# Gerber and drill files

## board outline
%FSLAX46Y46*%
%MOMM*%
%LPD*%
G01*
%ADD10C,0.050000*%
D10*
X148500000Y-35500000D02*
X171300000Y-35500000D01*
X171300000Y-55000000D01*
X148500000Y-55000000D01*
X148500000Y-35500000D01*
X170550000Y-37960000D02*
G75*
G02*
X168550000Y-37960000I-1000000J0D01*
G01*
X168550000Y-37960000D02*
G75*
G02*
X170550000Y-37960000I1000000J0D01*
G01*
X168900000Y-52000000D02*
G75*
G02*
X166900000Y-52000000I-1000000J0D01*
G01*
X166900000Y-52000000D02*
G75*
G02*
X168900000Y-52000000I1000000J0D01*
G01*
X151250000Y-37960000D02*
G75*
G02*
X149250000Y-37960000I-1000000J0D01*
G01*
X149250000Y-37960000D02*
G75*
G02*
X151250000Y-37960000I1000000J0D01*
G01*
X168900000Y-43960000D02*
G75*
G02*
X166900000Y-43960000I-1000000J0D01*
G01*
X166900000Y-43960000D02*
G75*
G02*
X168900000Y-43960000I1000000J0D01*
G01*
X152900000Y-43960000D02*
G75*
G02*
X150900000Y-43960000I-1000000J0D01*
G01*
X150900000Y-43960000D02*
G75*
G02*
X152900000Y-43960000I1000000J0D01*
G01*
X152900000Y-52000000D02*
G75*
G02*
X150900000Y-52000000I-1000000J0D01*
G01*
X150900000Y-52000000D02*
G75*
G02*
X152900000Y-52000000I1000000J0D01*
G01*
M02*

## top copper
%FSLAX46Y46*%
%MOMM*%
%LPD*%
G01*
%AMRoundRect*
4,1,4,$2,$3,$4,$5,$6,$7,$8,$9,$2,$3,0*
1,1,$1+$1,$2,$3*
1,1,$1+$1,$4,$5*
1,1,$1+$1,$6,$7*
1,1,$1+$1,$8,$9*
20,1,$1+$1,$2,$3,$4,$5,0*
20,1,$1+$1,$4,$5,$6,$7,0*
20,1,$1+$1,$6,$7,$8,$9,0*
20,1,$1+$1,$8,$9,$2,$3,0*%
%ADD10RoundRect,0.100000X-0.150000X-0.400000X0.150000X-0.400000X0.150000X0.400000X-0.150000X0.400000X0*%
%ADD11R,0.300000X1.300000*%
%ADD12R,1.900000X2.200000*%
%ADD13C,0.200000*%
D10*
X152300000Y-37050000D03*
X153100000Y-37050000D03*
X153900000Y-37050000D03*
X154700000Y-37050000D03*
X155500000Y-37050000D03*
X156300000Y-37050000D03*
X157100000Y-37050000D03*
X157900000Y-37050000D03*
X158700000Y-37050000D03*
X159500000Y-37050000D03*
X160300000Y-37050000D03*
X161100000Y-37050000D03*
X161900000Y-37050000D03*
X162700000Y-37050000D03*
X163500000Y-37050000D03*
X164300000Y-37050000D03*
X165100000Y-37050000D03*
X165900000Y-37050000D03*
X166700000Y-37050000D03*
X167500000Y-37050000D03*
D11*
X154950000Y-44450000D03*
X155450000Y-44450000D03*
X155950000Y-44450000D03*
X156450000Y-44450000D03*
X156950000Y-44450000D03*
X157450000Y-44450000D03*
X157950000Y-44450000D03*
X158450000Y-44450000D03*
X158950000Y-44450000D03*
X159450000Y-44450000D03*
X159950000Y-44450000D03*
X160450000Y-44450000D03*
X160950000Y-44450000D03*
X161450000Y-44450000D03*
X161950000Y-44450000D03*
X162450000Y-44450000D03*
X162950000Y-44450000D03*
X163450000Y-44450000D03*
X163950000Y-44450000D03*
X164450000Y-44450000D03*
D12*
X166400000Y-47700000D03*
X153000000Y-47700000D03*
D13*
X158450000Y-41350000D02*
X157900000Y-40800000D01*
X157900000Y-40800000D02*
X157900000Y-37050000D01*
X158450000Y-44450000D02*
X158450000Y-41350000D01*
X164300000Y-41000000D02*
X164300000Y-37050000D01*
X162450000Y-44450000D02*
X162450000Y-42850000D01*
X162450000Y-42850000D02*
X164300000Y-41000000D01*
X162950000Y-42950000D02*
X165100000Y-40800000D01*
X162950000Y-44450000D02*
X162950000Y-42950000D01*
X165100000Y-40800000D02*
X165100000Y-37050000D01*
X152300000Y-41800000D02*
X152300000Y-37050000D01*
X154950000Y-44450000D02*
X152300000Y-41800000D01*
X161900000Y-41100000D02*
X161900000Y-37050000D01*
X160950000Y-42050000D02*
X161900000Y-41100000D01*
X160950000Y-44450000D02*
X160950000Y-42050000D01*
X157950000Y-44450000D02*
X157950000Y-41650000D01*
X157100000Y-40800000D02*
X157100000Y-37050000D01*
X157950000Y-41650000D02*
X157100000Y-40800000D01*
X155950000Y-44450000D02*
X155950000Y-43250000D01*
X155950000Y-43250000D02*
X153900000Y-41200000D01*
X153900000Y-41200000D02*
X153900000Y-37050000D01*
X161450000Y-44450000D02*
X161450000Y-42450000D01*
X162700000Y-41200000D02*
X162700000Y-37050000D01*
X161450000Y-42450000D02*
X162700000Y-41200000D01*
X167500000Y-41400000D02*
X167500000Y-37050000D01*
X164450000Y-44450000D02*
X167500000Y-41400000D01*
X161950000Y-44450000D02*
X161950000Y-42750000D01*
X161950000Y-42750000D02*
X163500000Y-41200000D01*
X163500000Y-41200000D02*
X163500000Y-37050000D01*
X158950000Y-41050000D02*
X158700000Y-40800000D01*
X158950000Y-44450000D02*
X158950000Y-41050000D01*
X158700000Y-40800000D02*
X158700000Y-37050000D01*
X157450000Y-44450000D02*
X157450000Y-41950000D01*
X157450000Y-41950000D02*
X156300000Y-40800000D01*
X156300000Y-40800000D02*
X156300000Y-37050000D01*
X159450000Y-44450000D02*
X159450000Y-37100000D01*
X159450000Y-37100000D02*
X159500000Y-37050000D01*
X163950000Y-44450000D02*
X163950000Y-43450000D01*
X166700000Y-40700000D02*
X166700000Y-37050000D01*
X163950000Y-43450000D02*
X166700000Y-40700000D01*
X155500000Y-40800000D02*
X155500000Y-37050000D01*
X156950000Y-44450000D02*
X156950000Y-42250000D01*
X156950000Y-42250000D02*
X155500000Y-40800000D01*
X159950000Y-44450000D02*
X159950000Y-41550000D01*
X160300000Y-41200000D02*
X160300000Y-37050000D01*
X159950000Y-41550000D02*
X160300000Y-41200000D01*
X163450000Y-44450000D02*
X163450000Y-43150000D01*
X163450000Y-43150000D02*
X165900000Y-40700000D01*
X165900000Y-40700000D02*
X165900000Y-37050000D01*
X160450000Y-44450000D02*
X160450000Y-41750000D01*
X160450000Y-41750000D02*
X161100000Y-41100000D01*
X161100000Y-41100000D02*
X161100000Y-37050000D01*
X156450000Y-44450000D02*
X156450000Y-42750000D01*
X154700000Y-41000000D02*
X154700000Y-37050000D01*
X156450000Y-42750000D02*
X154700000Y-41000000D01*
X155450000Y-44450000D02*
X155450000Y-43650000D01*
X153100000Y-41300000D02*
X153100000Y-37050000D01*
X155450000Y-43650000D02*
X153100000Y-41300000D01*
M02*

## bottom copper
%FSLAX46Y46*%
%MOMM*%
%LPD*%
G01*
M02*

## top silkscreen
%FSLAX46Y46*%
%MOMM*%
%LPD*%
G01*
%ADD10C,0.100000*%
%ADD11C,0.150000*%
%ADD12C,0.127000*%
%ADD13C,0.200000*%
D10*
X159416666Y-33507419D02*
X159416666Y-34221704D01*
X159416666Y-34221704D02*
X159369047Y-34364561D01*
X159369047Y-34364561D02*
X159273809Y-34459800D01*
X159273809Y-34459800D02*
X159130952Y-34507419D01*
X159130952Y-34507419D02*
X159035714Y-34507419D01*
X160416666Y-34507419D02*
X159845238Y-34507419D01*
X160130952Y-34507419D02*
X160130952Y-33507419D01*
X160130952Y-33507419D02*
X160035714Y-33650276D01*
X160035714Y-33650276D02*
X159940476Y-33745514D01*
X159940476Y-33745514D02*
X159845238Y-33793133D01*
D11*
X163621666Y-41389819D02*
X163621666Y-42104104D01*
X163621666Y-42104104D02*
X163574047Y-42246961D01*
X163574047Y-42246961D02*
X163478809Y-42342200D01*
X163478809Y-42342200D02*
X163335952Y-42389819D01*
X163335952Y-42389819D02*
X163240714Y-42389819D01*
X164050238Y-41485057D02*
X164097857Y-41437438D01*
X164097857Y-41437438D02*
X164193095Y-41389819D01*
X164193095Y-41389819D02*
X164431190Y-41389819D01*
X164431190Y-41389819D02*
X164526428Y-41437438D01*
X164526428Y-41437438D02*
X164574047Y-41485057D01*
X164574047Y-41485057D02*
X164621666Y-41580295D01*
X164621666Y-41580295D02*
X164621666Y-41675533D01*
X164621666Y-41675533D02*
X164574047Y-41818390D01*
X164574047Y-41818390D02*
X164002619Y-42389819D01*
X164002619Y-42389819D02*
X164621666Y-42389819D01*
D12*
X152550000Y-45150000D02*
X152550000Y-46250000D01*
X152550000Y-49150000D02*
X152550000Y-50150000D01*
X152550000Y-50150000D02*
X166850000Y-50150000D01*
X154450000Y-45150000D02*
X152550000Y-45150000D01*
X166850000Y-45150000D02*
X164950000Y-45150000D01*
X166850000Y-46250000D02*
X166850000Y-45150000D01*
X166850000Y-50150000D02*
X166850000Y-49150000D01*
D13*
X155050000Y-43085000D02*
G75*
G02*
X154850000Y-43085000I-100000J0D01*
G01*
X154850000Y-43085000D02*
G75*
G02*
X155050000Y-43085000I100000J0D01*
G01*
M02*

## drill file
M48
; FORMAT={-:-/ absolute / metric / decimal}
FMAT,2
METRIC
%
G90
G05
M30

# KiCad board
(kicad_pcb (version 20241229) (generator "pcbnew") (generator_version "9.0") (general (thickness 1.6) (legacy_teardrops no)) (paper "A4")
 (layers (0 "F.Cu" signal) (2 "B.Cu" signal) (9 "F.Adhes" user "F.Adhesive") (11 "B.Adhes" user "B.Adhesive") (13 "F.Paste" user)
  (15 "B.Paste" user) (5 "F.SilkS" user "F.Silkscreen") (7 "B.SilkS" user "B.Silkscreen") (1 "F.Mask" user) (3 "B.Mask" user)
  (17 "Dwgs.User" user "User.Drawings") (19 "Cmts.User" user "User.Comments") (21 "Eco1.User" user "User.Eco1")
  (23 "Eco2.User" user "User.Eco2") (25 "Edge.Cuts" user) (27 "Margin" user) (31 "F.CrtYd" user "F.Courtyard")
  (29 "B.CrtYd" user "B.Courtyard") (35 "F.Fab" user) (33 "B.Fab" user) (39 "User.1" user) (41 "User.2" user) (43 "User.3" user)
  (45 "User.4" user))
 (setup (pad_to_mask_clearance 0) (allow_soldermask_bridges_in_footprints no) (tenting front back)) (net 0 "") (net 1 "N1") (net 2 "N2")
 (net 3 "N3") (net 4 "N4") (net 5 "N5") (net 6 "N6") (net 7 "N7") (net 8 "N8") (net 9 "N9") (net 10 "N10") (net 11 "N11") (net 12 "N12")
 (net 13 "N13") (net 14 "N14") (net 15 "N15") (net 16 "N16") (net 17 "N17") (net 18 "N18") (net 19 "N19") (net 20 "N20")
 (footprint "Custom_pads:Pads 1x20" (layer "F.Cu") (at 159.75 37.05)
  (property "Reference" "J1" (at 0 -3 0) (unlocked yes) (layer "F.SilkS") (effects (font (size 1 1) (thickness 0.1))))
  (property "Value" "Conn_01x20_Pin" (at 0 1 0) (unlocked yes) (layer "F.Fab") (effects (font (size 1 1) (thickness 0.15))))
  (pad "1" smd roundrect (at -7.45 0) (size 0.5 1) (layers "F.Cu" "F.Mask" "F.Paste") (roundrect_rratio 0.2) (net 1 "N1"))
  (pad "2" smd roundrect (at -6.65 0) (size 0.5 1) (layers "F.Cu" "F.Mask" "F.Paste") (roundrect_rratio 0.2) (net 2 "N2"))
  (pad "3" smd roundrect (at -5.85 0) (size 0.5 1) (layers "F.Cu" "F.Mask" "F.Paste") (roundrect_rratio 0.2) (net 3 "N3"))
  (pad "4" smd roundrect (at -5.05 0) (size 0.5 1) (layers "F.Cu" "F.Mask" "F.Paste") (roundrect_rratio 0.2) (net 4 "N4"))
  (pad "5" smd roundrect (at -4.25 0) (size 0.5 1) (layers "F.Cu" "F.Mask" "F.Paste") (roundrect_rratio 0.2) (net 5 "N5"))
  (pad "6" smd roundrect (at -3.45 0) (size 0.5 1) (layers "F.Cu" "F.Mask" "F.Paste") (roundrect_rratio 0.2) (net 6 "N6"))
  (pad "7" smd roundrect (at -2.65 0) (size 0.5 1) (layers "F.Cu" "F.Mask" "F.Paste") (roundrect_rratio 0.2) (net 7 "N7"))
  (pad "8" smd roundrect (at -1.85 0) (size 0.5 1) (layers "F.Cu" "F.Mask" "F.Paste") (roundrect_rratio 0.2) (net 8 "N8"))
  (pad "9" smd roundrect (at -1.05 0) (size 0.5 1) (layers "F.Cu" "F.Mask" "F.Paste") (roundrect_rratio 0.2) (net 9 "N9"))
  (pad "10" smd roundrect (at -0.25 0) (size 0.5 1) (layers "F.Cu" "F.Mask" "F.Paste") (roundrect_rratio 0.2) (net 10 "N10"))
  (pad "11" smd roundrect (at 0.55 0) (size 0.5 1) (layers "F.Cu" "F.Mask" "F.Paste") (roundrect_rratio 0.2) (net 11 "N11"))
  (pad "12" smd roundrect (at 1.35 0) (size 0.5 1) (layers "F.Cu" "F.Mask" "F.Paste") (roundrect_rratio 0.2) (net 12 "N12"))
  (pad "13" smd roundrect (at 2.15 0) (size 0.5 1) (layers "F.Cu" "F.Mask" "F.Paste") (roundrect_rratio 0.2) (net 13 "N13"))
  (pad "14" smd roundrect (at 2.95 0) (size 0.5 1) (layers "F.Cu" "F.Mask" "F.Paste") (roundrect_rratio 0.2) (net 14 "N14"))
  (pad "15" smd roundrect (at 3.75 0) (size 0.5 1) (layers "F.Cu" "F.Mask" "F.Paste") (roundrect_rratio 0.2) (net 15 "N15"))
  (pad "16" smd roundrect (at 4.55 0) (size 0.5 1) (layers "F.Cu" "F.Mask" "F.Paste") (roundrect_rratio 0.2) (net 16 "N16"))
  (pad "17" smd roundrect (at 5.35 0) (size 0.5 1) (layers "F.Cu" "F.Mask" "F.Paste") (roundrect_rratio 0.2) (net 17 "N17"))
  (pad "18" smd roundrect (at 6.15 0) (size 0.5 1) (layers "F.Cu" "F.Mask" "F.Paste") (roundrect_rratio 0.2) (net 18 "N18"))
  (pad "19" smd roundrect (at 6.95 0) (size 0.5 1) (layers "F.Cu" "F.Mask" "F.Paste") (roundrect_rratio 0.2) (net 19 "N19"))
  (pad "20" smd roundrect (at 7.75 0) (size 0.5 1) (layers "F.Cu" "F.Mask" "F.Paste") (roundrect_rratio 0.2) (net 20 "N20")))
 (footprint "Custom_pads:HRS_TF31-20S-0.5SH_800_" (layer "F.Cu") (at 159.7 47.65 180)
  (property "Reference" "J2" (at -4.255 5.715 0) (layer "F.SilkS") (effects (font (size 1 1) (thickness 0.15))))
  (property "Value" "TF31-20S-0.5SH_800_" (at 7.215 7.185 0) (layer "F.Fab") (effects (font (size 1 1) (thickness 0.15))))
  (fp_line (start 7.15 2.5) (end 7.15 1.4) (stroke (width 0.127) (type solid)) (layer "F.SilkS"))
  (fp_line (start 7.15 -1.5) (end 7.15 -2.5) (stroke (width 0.127) (type solid)) (layer "F.SilkS"))
  (fp_line (start 7.15 -2.5) (end -7.15 -2.5) (stroke (width 0.127) (type solid)) (layer "F.SilkS"))
  (fp_line (start 5.25 2.5) (end 7.15 2.5) (stroke (width 0.127) (type solid)) (layer "F.SilkS"))
  (fp_line (start -7.15 2.5) (end -5.25 2.5) (stroke (width 0.127) (type solid)) (layer "F.SilkS"))
  (fp_line (start -7.15 1.4) (end -7.15 2.5) (stroke (width 0.127) (type solid)) (layer "F.SilkS"))
  (fp_line (start -7.15 -2.5) (end -7.15 -1.5) (stroke (width 0.127) (type solid)) (layer "F.SilkS"))
  (fp_circle (center 4.75 4.565) (end 4.85 4.565) (stroke (width 0.2) (type solid)) (fill no) (layer "F.SilkS"))
  (pad "1" smd rect (at 4.75 3.2 180) (size 0.3 1.3) (layers "F.Cu" "F.Mask" "F.Paste") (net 1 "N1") (solder_mask_margin 0.102))
  (pad "2" smd rect (at 4.25 3.2 180) (size 0.3 1.3) (layers "F.Cu" "F.Mask" "F.Paste") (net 2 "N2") (solder_mask_margin 0.102))
  (pad "3" smd rect (at 3.75 3.2 180) (size 0.3 1.3) (layers "F.Cu" "F.Mask" "F.Paste") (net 3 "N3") (solder_mask_margin 0.102))
  (pad "4" smd rect (at 3.25 3.2 180) (size 0.3 1.3) (layers "F.Cu" "F.Mask" "F.Paste") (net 4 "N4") (solder_mask_margin 0.102))
  (pad "5" smd rect (at 2.75 3.2 180) (size 0.3 1.3) (layers "F.Cu" "F.Mask" "F.Paste") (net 5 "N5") (solder_mask_margin 0.102))
  (pad "6" smd rect (at 2.25 3.2 180) (size 0.3 1.3) (layers "F.Cu" "F.Mask" "F.Paste") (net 6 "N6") (solder_mask_margin 0.102))
  (pad "7" smd rect (at 1.75 3.2 180) (size 0.3 1.3) (layers "F.Cu" "F.Mask" "F.Paste") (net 7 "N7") (solder_mask_margin 0.102))
  (pad "8" smd rect (at 1.25 3.2 180) (size 0.3 1.3) (layers "F.Cu" "F.Mask" "F.Paste") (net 8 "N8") (solder_mask_margin 0.102))
  (pad "9" smd rect (at 0.75 3.2 180) (size 0.3 1.3) (layers "F.Cu" "F.Mask" "F.Paste") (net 9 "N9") (solder_mask_margin 0.102))
  (pad "10" smd rect (at 0.25 3.2 180) (size 0.3 1.3) (layers "F.Cu" "F.Mask" "F.Paste") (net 10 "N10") (solder_mask_margin 0.102))
  (pad "11" smd rect (at -0.25 3.2 180) (size 0.3 1.3) (layers "F.Cu" "F.Mask" "F.Paste") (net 11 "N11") (solder_mask_margin 0.102))
  (pad "12" smd rect (at -0.75 3.2 180) (size 0.3 1.3) (layers "F.Cu" "F.Mask" "F.Paste") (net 12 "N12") (solder_mask_margin 0.102))
  (pad "13" smd rect (at -1.25 3.2 180) (size 0.3 1.3) (layers "F.Cu" "F.Mask" "F.Paste") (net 13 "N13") (solder_mask_margin 0.102))
  (pad "14" smd rect (at -1.75 3.2 180) (size 0.3 1.3) (layers "F.Cu" "F.Mask" "F.Paste") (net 14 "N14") (solder_mask_margin 0.102))
  (pad "15" smd rect (at -2.25 3.2 180) (size 0.3 1.3) (layers "F.Cu" "F.Mask" "F.Paste") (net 15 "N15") (solder_mask_margin 0.102))
  (pad "16" smd rect (at -2.75 3.2 180) (size 0.3 1.3) (layers "F.Cu" "F.Mask" "F.Paste") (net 16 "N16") (solder_mask_margin 0.102))
  (pad "17" smd rect (at -3.25 3.2 180) (size 0.3 1.3) (layers "F.Cu" "F.Mask" "F.Paste") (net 17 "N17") (solder_mask_margin 0.102))
  (pad "18" smd rect (at -3.75 3.2 180) (size 0.3 1.3) (layers "F.Cu" "F.Mask" "F.Paste") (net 18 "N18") (solder_mask_margin 0.102))
  (pad "19" smd rect (at -4.25 3.2 180) (size 0.3 1.3) (layers "F.Cu" "F.Mask" "F.Paste") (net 19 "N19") (solder_mask_margin 0.102))
  (pad "20" smd rect (at -4.75 3.2 180) (size 0.3 1.3) (layers "F.Cu" "F.Mask" "F.Paste") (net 20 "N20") (solder_mask_margin 0.102))
  (pad "S1" smd rect (at -6.7 -0.05 180) (size 1.9 2.2) (layers "F.Cu" "F.Mask" "F.Paste") (solder_mask_margin 0.102))
  (pad "S2" smd rect (at 6.7 -0.05 180) (size 1.9 2.2) (layers "F.Cu" "F.Mask" "F.Paste") (solder_mask_margin 0.102)))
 (gr_rect (start 148.5 35.5) (end 171.3 55) (stroke (width 0.05) (type solid)) (fill no) (layer "Edge.Cuts"))
 (gr_circle (center 169.55 37.96) (end 170.55 37.96) (stroke (width 0.05) (type default)) (fill no) (layer "Edge.Cuts"))
 (gr_circle (center 167.9 52) (end 168.9 52) (stroke (width 0.05) (type default)) (fill no) (layer "Edge.Cuts"))
 (gr_circle (center 150.25 37.96) (end 151.25 37.96) (stroke (width 0.05) (type default)) (fill no) (layer "Edge.Cuts"))
 (gr_circle (center 167.9 43.96) (end 168.9 43.96) (stroke (width 0.05) (type default)) (fill no) (layer "Edge.Cuts"))
 (gr_circle (center 151.9 43.96) (end 152.9 43.96) (stroke (width 0.05) (type default)) (fill no) (layer "Edge.Cuts"))
 (gr_circle (center 151.9 52) (end 152.9 52) (stroke (width 0.05) (type default)) (fill no) (layer "Edge.Cuts"))
 (segment (start 158.45 41.35) (end 157.9 40.8) (width 0.2) (layer "F.Cu") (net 8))
 (segment (start 157.9 40.8) (end 157.9 37.05) (width 0.2) (layer "F.Cu") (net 8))
 (segment (start 158.45 44.45) (end 158.45 41.35) (width 0.2) (layer "F.Cu") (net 8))
 (segment (start 164.3 41) (end 164.3 37.05) (width 0.2) (layer "F.Cu") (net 16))
 (segment (start 162.45 44.45) (end 162.45 42.85) (width 0.2) (layer "F.Cu") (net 16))
 (segment (start 162.45 42.85) (end 164.3 41) (width 0.2) (layer "F.Cu") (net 16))
 (segment (start 162.95 42.95) (end 165.1 40.8) (width 0.2) (layer "F.Cu") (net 17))
 (segment (start 162.95 44.45) (end 162.95 42.95) (width 0.2) (layer "F.Cu") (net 17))
 (segment (start 165.1 40.8) (end 165.1 37.05) (width 0.2) (layer "F.Cu") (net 17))
 (segment (start 152.3 41.8) (end 152.3 37.05) (width 0.2) (layer "F.Cu") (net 1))
 (segment (start 154.95 44.45) (end 152.3 41.8) (width 0.2) (layer "F.Cu") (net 1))
 (segment (start 161.9 41.1) (end 161.9 37.05) (width 0.2) (layer "F.Cu") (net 13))
 (segment (start 160.95 42.05) (end 161.9 41.1) (width 0.2) (layer "F.Cu") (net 13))
 (segment (start 160.95 44.45) (end 160.95 42.05) (width 0.2) (layer "F.Cu") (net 13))
 (segment (start 157.95 44.45) (end 157.95 41.65) (width 0.2) (layer "F.Cu") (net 7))
 (segment (start 157.1 40.8) (end 157.1 37.05) (width 0.2) (layer "F.Cu") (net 7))
 (segment (start 157.95 41.65) (end 157.1 40.8) (width 0.2) (layer "F.Cu") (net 7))
 (segment (start 155.95 44.45) (end 155.95 43.25) (width 0.2) (layer "F.Cu") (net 3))
 (segment (start 155.95 43.25) (end 153.9 41.2) (width 0.2) (layer "F.Cu") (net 3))
 (segment (start 153.9 41.2) (end 153.9 37.05) (width 0.2) (layer "F.Cu") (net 3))
 (segment (start 161.45 44.45) (end 161.45 42.45) (width 0.2) (layer "F.Cu") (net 14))
 (segment (start 162.7 41.2) (end 162.7 37.05) (width 0.2) (layer "F.Cu") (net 14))
 (segment (start 161.45 42.45) (end 162.7 41.2) (width 0.2) (layer "F.Cu") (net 14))
 (segment (start 167.5 41.4) (end 167.5 37.05) (width 0.2) (layer "F.Cu") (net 20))
 (segment (start 164.45 44.45) (end 167.5 41.4) (width 0.2) (layer "F.Cu") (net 20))
 (segment (start 161.95 44.45) (end 161.95 42.75) (width 0.2) (layer "F.Cu") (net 15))
 (segment (start 161.95 42.75) (end 163.5 41.2) (width 0.2) (layer "F.Cu") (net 15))
 (segment (start 163.5 41.2) (end 163.5 37.05) (width 0.2) (layer "F.Cu") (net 15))
 (segment (start 158.95 41.05) (end 158.7 40.8) (width 0.2) (layer "F.Cu") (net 9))
 (segment (start 158.95 44.45) (end 158.95 41.05) (width 0.2) (layer "F.Cu") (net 9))
 (segment (start 158.7 40.8) (end 158.7 37.05) (width 0.2) (layer "F.Cu") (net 9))
 (segment (start 157.45 44.45) (end 157.45 41.95) (width 0.2) (layer "F.Cu") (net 6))
 (segment (start 157.45 41.95) (end 156.3 40.8) (width 0.2) (layer "F.Cu") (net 6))
 (segment (start 156.3 40.8) (end 156.3 37.05) (width 0.2) (layer "F.Cu") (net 6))
 (segment (start 159.45 44.45) (end 159.45 37.1) (width 0.2) (layer "F.Cu") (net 10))
 (segment (start 159.45 37.1) (end 159.5 37.05) (width 0.2) (layer "F.Cu") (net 10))
 (segment (start 163.95 44.45) (end 163.95 43.45) (width 0.2) (layer "F.Cu") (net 19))
 (segment (start 166.7 40.7) (end 166.7 37.05) (width 0.2) (layer "F.Cu") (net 19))
 (segment (start 163.95 43.45) (end 166.7 40.7) (width 0.2) (layer "F.Cu") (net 19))
 (segment (start 155.5 40.8) (end 155.5 37.05) (width 0.2) (layer "F.Cu") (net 5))
 (segment (start 156.95 44.45) (end 156.95 42.25) (width 0.2) (layer "F.Cu") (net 5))
 (segment (start 156.95 42.25) (end 155.5 40.8) (width 0.2) (layer "F.Cu") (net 5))
 (segment (start 159.95 44.45) (end 159.95 41.55) (width 0.2) (layer "F.Cu") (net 11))
 (segment (start 160.3 41.2) (end 160.3 37.05) (width 0.2) (layer "F.Cu") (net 11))
 (segment (start 159.95 41.55) (end 160.3 41.2) (width 0.2) (layer "F.Cu") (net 11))
 (segment (start 163.45 44.45) (end 163.45 43.15) (width 0.2) (layer "F.Cu") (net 18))
 (segment (start 163.45 43.15) (end 165.9 40.7) (width 0.2) (layer "F.Cu") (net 18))
 (segment (start 165.9 40.7) (end 165.9 37.05) (width 0.2) (layer "F.Cu") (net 18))
 (segment (start 160.45 44.45) (end 160.45 41.75) (width 0.2) (layer "F.Cu") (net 12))
 (segment (start 160.45 41.75) (end 161.1 41.1) (width 0.2) (layer "F.Cu") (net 12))
 (segment (start 161.1 41.1) (end 161.1 37.05) (width 0.2) (layer "F.Cu") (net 12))
 (segment (start 156.45 44.45) (end 156.45 42.75) (width 0.2) (layer "F.Cu") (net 4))
 (segment (start 154.7 41) (end 154.7 37.05) (width 0.2) (layer "F.Cu") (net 4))
 (segment (start 156.45 42.75) (end 154.7 41) (width 0.2) (layer "F.Cu") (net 4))
 (segment (start 155.45 44.45) (end 155.45 43.65) (width 0.2) (layer "F.Cu") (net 2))
 (segment (start 153.1 41.3) (end 153.1 37.05) (width 0.2) (layer "F.Cu") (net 2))
 (segment (start 155.45 43.65) (end 153.1 41.3) (width 0.2) (layer "F.Cu") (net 2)))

